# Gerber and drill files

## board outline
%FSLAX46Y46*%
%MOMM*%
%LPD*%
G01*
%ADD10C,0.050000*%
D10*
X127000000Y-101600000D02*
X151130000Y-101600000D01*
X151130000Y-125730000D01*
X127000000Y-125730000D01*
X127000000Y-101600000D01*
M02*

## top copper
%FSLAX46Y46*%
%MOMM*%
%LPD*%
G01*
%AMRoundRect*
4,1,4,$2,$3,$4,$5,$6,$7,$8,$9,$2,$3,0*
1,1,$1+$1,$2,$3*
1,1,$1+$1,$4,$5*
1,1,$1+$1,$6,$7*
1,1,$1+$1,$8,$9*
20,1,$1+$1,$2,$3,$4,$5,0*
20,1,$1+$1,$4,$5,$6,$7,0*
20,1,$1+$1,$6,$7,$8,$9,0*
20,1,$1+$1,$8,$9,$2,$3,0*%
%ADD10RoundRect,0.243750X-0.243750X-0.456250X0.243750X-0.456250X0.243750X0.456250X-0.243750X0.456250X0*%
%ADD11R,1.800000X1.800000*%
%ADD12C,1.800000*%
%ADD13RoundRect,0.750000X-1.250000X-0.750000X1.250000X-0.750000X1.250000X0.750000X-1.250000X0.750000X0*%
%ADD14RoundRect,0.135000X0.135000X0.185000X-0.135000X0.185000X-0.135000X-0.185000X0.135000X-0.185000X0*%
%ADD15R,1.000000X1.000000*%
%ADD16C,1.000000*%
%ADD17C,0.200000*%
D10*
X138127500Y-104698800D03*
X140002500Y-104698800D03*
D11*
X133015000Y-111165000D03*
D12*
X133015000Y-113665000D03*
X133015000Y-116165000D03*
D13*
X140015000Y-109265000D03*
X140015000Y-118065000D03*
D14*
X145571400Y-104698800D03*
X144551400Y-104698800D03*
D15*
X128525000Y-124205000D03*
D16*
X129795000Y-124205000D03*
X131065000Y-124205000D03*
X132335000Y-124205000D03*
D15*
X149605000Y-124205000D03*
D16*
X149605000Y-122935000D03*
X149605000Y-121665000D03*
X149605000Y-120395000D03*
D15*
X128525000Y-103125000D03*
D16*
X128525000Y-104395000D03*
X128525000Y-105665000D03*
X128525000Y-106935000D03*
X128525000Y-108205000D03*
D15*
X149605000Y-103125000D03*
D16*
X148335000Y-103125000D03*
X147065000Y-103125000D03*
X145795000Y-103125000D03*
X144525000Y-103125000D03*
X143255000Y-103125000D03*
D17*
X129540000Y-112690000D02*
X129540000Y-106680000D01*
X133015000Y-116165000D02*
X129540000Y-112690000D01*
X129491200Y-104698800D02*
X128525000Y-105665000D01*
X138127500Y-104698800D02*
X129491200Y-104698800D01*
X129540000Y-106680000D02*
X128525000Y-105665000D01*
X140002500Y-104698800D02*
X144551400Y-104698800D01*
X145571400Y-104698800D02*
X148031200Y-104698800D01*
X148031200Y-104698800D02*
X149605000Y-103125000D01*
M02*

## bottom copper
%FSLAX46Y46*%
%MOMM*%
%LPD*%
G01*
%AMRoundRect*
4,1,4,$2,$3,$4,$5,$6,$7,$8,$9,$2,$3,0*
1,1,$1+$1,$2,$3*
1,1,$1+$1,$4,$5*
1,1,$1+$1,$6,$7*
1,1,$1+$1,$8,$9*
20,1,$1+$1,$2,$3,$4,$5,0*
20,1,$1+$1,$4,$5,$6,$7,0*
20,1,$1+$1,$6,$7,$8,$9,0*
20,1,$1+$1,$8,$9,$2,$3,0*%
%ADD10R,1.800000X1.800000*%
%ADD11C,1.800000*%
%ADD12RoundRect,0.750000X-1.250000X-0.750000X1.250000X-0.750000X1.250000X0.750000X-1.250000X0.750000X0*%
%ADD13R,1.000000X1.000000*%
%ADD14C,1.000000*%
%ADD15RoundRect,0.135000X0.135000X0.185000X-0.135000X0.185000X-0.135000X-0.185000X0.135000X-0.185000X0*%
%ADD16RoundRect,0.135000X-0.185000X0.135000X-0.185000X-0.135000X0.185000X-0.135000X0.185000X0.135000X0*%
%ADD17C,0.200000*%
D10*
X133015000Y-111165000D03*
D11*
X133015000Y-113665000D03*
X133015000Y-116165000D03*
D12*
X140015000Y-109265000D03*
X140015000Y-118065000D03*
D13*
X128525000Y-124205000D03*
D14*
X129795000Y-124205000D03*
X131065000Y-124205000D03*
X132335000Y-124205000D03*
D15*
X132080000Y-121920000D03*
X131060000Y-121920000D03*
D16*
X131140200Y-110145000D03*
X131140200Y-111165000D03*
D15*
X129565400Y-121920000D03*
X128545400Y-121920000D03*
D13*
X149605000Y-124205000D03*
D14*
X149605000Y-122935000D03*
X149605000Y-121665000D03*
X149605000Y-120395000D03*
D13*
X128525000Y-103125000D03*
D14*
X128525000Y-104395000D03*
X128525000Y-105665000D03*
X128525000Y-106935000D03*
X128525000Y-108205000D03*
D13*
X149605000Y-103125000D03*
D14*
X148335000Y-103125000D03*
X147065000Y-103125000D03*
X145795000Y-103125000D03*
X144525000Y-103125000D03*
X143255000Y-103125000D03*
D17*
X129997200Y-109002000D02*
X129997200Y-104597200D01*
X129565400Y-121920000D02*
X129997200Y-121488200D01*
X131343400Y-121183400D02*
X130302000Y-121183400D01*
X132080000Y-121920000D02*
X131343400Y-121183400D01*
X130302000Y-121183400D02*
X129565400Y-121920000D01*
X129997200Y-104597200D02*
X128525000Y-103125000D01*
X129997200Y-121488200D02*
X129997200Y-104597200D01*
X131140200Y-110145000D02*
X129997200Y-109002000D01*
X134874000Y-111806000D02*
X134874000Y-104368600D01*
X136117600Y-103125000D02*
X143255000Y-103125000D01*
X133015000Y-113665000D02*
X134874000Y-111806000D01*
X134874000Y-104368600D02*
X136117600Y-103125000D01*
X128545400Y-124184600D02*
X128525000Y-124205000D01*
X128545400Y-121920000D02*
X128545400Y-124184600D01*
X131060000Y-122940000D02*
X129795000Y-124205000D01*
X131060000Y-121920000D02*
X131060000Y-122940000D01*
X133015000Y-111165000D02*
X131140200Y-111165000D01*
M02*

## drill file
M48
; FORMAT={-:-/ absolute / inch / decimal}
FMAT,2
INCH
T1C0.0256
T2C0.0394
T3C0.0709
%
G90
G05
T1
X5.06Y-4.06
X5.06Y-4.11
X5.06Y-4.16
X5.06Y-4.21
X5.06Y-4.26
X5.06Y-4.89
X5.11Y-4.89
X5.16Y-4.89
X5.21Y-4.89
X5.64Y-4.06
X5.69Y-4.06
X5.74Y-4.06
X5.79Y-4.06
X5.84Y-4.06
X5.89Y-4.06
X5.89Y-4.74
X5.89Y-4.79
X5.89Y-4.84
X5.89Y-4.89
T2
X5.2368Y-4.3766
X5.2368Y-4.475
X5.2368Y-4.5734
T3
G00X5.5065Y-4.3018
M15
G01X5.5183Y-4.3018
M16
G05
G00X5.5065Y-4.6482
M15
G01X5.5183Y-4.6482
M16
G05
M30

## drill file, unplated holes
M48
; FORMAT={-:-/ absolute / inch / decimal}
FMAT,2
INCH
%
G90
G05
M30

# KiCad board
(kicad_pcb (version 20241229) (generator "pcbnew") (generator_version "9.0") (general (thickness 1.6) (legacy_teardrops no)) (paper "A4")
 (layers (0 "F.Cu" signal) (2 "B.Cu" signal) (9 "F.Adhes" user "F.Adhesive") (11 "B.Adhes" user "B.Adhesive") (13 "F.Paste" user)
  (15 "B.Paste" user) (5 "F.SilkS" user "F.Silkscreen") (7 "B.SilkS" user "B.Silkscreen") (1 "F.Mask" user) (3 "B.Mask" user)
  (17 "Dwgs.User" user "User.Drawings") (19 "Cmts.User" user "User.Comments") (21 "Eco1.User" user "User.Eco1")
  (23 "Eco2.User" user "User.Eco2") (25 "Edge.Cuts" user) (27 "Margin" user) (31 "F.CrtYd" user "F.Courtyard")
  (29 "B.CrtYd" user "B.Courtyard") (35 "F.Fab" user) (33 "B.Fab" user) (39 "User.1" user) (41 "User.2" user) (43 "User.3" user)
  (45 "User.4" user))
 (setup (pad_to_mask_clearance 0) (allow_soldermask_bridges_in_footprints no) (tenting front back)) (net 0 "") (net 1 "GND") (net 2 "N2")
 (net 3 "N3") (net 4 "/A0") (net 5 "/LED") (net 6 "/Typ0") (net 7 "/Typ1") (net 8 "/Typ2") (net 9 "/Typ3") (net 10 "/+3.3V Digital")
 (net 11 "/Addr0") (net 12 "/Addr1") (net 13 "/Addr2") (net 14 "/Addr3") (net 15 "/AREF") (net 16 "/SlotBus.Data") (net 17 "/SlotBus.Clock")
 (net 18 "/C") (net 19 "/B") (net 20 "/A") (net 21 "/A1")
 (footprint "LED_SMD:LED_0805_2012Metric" (layer "F.Cu") (at 139.065 104.6988)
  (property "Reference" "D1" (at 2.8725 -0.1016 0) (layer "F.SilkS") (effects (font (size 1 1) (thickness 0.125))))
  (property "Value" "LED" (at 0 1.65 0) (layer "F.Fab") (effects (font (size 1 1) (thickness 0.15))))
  (pad "1" smd roundrect (at -0.9375 0) (size 0.975 1.4) (layers "F.Cu" "F.Mask" "F.Paste") (roundrect_rratio 0.25) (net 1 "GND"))
  (pad "2" smd roundrect (at 0.9375 0) (size 0.975 1.4) (layers "F.Cu" "F.Mask" "F.Paste") (roundrect_rratio 0.25) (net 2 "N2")))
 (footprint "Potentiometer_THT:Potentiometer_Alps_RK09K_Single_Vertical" (layer "F.Cu") (at 133.015 111.165)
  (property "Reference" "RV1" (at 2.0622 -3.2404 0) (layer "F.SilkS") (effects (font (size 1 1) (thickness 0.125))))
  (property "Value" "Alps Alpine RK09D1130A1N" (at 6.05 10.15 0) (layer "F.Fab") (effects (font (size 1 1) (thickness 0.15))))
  (pad "1" thru_hole rect (at 0 0) (size 1.8 1.8) (drill 1) (layers "*.Cu" "*.Mask") (remove_unused_layers no) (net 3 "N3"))
  (pad "2" thru_hole circle (at 0 2.5) (size 1.8 1.8) (drill 1) (layers "*.Cu" "*.Mask") (remove_unused_layers no) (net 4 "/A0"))
  (pad "3" thru_hole circle (at 0 5) (size 1.8 1.8) (drill 1) (layers "*.Cu" "*.Mask") (remove_unused_layers no) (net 1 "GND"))
  (pad "MP" thru_hole roundrect (at 7 -1.9) (size 4 3) (drill oval 2.1 1.8) (layers "*.Cu" "*.Mask") (remove_unused_layers no)
   (roundrect_rratio 0.25))
  (pad "MP" thru_hole roundrect (at 7 6.9) (size 4 3) (drill oval 2.1 1.8) (layers "*.Cu" "*.Mask") (remove_unused_layers no)
   (roundrect_rratio 0.25)))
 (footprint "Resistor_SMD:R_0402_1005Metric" (layer "F.Cu") (at 145.0614 104.6988 180)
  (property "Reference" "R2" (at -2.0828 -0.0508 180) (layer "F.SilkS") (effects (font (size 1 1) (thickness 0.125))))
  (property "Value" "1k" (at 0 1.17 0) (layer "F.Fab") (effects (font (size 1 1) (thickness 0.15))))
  (pad "1" smd roundrect (at -0.51 0 180) (size 0.54 0.64) (layers "F.Cu" "F.Mask" "F.Paste") (roundrect_rratio 0.25) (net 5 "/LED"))
  (pad "2" smd roundrect (at 0.51 0 180) (size 0.54 0.64) (layers "F.Cu" "F.Mask" "F.Paste") (roundrect_rratio 0.25) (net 2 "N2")))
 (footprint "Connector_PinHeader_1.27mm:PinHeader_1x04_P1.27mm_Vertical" (layer "B.Cu") (at 128.525 124.205 -90)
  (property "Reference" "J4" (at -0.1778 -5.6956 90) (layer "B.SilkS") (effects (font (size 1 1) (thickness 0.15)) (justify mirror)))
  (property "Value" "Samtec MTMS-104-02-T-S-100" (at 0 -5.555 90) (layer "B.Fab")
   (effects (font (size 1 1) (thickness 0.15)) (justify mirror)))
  (pad "1" thru_hole rect (at 0 0 270) (size 1 1) (drill 0.65) (layers "*.Cu" "*.Mask") (remove_unused_layers no) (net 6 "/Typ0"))
  (pad "2" thru_hole circle (at 0 -1.27 270) (size 1 1) (drill 0.65) (layers "*.Cu" "*.Mask") (remove_unused_layers no) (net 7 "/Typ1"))
  (pad "3" thru_hole circle (at 0 -2.54 270) (size 1 1) (drill 0.65) (layers "*.Cu" "*.Mask") (remove_unused_layers no) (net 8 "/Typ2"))
  (pad "4" thru_hole circle (at 0 -3.81 270) (size 1 1) (drill 0.65) (layers "*.Cu" "*.Mask") (remove_unused_layers no) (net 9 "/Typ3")))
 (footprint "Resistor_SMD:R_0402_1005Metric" (layer "B.Cu") (at 131.57 121.92 180)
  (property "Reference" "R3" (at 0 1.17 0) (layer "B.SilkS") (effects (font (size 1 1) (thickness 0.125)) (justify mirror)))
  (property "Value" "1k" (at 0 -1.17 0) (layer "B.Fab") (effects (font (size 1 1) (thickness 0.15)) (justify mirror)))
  (pad "1" smd roundrect (at -0.51 0 180) (size 0.54 0.64) (layers "B.Cu" "B.Mask" "B.Paste") (roundrect_rratio 0.25)
   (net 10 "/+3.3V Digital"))
  (pad "2" smd roundrect (at 0.51 0 180) (size 0.54 0.64) (layers "B.Cu" "B.Mask" "B.Paste") (roundrect_rratio 0.25) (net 7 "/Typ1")))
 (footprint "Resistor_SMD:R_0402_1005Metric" (layer "B.Cu") (at 131.1402 110.655 -90)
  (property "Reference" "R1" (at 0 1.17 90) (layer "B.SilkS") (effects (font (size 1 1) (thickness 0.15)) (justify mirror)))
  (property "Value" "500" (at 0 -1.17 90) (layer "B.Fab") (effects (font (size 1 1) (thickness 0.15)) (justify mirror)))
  (pad "1" smd roundrect (at -0.51 0 270) (size 0.54 0.64) (layers "B.Cu" "B.Mask" "B.Paste") (roundrect_rratio 0.25)
   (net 10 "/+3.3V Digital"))
  (pad "2" smd roundrect (at 0.51 0 270) (size 0.54 0.64) (layers "B.Cu" "B.Mask" "B.Paste") (roundrect_rratio 0.25) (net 3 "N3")))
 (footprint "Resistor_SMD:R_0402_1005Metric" (layer "B.Cu") (at 129.0554 121.92 180)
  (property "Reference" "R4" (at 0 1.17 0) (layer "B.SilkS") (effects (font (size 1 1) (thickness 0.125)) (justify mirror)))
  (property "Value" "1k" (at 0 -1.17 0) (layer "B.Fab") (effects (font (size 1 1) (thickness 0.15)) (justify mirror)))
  (pad "1" smd roundrect (at -0.51 0 180) (size 0.54 0.64) (layers "B.Cu" "B.Mask" "B.Paste") (roundrect_rratio 0.25)
   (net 10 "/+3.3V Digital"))
  (pad "2" smd roundrect (at 0.51 0 180) (size 0.54 0.64) (layers "B.Cu" "B.Mask" "B.Paste") (roundrect_rratio 0.25) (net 6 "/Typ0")))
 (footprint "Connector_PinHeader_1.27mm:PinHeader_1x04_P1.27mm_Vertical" (layer "B.Cu") (at 149.605 124.205)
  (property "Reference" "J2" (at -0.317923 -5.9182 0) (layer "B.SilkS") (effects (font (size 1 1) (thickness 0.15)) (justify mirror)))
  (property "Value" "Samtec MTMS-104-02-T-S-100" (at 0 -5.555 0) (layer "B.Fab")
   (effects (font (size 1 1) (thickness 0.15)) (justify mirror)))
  (pad "1" thru_hole rect (at 0 0) (size 1 1) (drill 0.65) (layers "*.Cu" "*.Mask") (remove_unused_layers no) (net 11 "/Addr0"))
  (pad "2" thru_hole circle (at 0 -1.27) (size 1 1) (drill 0.65) (layers "*.Cu" "*.Mask") (remove_unused_layers no) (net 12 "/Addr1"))
  (pad "3" thru_hole circle (at 0 -2.54) (size 1 1) (drill 0.65) (layers "*.Cu" "*.Mask") (remove_unused_layers no) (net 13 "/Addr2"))
  (pad "4" thru_hole circle (at 0 -3.81) (size 1 1) (drill 0.65) (layers "*.Cu" "*.Mask") (remove_unused_layers no) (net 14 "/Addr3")))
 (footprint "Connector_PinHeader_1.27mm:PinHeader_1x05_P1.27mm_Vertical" (layer "B.Cu") (at 128.525 103.125 180)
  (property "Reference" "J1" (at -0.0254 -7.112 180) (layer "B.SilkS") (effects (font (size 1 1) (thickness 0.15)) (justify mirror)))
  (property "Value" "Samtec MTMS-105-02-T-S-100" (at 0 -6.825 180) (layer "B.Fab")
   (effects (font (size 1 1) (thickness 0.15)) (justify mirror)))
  (pad "1" thru_hole rect (at 0 0 180) (size 1 1) (drill 0.65) (layers "*.Cu" "*.Mask") (remove_unused_layers no) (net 10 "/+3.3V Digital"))
  (pad "2" thru_hole circle (at 0 -1.27 180) (size 1 1) (drill 0.65) (layers "*.Cu" "*.Mask") (remove_unused_layers no) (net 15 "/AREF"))
  (pad "3" thru_hole circle (at 0 -2.54 180) (size 1 1) (drill 0.65) (layers "*.Cu" "*.Mask") (remove_unused_layers no) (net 1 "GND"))
  (pad "4" thru_hole circle (at 0 -3.81 180) (size 1 1) (drill 0.65) (layers "*.Cu" "*.Mask") (remove_unused_layers no)
   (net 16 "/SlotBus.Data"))
  (pad "5" thru_hole circle (at 0 -5.08 180) (size 1 1) (drill 0.65) (layers "*.Cu" "*.Mask") (remove_unused_layers no)
   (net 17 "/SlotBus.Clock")))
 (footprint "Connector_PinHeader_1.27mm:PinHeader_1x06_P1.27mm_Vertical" (layer "B.Cu") (at 149.605 103.125 90)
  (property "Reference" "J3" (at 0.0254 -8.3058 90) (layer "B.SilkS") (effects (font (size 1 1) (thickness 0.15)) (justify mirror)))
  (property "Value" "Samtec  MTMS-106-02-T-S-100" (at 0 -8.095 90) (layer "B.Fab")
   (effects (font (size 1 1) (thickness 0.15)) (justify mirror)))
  (pad "1" thru_hole rect (at 0 0 90) (size 1 1) (drill 0.65) (layers "*.Cu" "*.Mask") (remove_unused_layers no) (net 5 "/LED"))
  (pad "2" thru_hole circle (at 0 -1.27 90) (size 1 1) (drill 0.65) (layers "*.Cu" "*.Mask") (remove_unused_layers no) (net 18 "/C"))
  (pad "3" thru_hole circle (at 0 -2.54 90) (size 1 1) (drill 0.65) (layers "*.Cu" "*.Mask") (remove_unused_layers no) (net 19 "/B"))
  (pad "4" thru_hole circle (at 0 -3.81 90) (size 1 1) (drill 0.65) (layers "*.Cu" "*.Mask") (remove_unused_layers no) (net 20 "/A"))
  (pad "5" thru_hole circle (at 0 -5.08 90) (size 1 1) (drill 0.65) (layers "*.Cu" "*.Mask") (remove_unused_layers no) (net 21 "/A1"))
  (pad "6" thru_hole circle (at 0 -6.35 90) (size 1 1) (drill 0.65) (layers "*.Cu" "*.Mask") (remove_unused_layers no) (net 4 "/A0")))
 (gr_rect (start 127 101.6) (end 151.13 125.73) (stroke (width 0.05) (type solid)) (fill no) (layer "Edge.Cuts"))
 (segment (start 129.54 112.69) (end 129.54 106.68) (width 0.2) (layer "F.Cu") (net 1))
 (segment (start 133.015 116.165) (end 129.54 112.69) (width 0.2) (layer "F.Cu") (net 1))
 (segment (start 129.4912 104.6988) (end 128.525 105.665) (width 0.2) (layer "F.Cu") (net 1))
 (segment (start 138.1275 104.6988) (end 129.4912 104.6988) (width 0.2) (layer "F.Cu") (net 1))
 (segment (start 129.54 106.68) (end 128.525 105.665) (width 0.2) (layer "F.Cu") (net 1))
 (segment (start 140.0025 104.6988) (end 144.5514 104.6988) (width 0.2) (layer "F.Cu") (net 2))
 (segment (start 129.9972 109.002) (end 129.9972 104.5972) (width 0.2) (layer "B.Cu") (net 10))
 (segment (start 129.5654 121.92) (end 129.9972 121.4882) (width 0.2) (layer "B.Cu") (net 10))
 (segment (start 131.3434 121.1834) (end 130.302 121.1834) (width 0.2) (layer "B.Cu") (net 10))
 (segment (start 132.08 121.92) (end 131.3434 121.1834) (width 0.2) (layer "B.Cu") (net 10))
 (segment (start 130.302 121.1834) (end 129.5654 121.92) (width 0.2) (layer "B.Cu") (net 10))
 (segment (start 129.9972 104.5972) (end 128.525 103.125) (width 0.2) (layer "B.Cu") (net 10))
 (segment (start 129.9972 121.4882) (end 129.9972 104.5972) (width 0.2) (layer "B.Cu") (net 10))
 (segment (start 131.1402 110.145) (end 129.9972 109.002) (width 0.2) (layer "B.Cu") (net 10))
 (segment (start 145.5714 104.6988) (end 148.0312 104.6988) (width 0.2) (layer "F.Cu") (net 5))
 (segment (start 148.0312 104.6988) (end 149.605 103.125) (width 0.2) (layer "F.Cu") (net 5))
 (segment (start 134.874 111.806) (end 134.874 104.3686) (width 0.2) (layer "B.Cu") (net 4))
 (segment (start 136.1176 103.125) (end 143.255 103.125) (width 0.2) (layer "B.Cu") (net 4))
 (segment (start 133.015 113.665) (end 134.874 111.806) (width 0.2) (layer "B.Cu") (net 4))
 (segment (start 134.874 104.3686) (end 136.1176 103.125) (width 0.2) (layer "B.Cu") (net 4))
 (segment (start 128.5454 124.1846) (end 128.525 124.205) (width 0.2) (layer "B.Cu") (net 6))
 (segment (start 128.5454 121.92) (end 128.5454 124.1846) (width 0.2) (layer "B.Cu") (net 6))
 (segment (start 131.06 122.94) (end 129.795 124.205) (width 0.2) (layer "B.Cu") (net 7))
 (segment (start 131.06 121.92) (end 131.06 122.94) (width 0.2) (layer "B.Cu") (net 7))
 (segment (start 133.015 111.165) (end 131.1402 111.165) (width 0.2) (layer "B.Cu") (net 3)))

